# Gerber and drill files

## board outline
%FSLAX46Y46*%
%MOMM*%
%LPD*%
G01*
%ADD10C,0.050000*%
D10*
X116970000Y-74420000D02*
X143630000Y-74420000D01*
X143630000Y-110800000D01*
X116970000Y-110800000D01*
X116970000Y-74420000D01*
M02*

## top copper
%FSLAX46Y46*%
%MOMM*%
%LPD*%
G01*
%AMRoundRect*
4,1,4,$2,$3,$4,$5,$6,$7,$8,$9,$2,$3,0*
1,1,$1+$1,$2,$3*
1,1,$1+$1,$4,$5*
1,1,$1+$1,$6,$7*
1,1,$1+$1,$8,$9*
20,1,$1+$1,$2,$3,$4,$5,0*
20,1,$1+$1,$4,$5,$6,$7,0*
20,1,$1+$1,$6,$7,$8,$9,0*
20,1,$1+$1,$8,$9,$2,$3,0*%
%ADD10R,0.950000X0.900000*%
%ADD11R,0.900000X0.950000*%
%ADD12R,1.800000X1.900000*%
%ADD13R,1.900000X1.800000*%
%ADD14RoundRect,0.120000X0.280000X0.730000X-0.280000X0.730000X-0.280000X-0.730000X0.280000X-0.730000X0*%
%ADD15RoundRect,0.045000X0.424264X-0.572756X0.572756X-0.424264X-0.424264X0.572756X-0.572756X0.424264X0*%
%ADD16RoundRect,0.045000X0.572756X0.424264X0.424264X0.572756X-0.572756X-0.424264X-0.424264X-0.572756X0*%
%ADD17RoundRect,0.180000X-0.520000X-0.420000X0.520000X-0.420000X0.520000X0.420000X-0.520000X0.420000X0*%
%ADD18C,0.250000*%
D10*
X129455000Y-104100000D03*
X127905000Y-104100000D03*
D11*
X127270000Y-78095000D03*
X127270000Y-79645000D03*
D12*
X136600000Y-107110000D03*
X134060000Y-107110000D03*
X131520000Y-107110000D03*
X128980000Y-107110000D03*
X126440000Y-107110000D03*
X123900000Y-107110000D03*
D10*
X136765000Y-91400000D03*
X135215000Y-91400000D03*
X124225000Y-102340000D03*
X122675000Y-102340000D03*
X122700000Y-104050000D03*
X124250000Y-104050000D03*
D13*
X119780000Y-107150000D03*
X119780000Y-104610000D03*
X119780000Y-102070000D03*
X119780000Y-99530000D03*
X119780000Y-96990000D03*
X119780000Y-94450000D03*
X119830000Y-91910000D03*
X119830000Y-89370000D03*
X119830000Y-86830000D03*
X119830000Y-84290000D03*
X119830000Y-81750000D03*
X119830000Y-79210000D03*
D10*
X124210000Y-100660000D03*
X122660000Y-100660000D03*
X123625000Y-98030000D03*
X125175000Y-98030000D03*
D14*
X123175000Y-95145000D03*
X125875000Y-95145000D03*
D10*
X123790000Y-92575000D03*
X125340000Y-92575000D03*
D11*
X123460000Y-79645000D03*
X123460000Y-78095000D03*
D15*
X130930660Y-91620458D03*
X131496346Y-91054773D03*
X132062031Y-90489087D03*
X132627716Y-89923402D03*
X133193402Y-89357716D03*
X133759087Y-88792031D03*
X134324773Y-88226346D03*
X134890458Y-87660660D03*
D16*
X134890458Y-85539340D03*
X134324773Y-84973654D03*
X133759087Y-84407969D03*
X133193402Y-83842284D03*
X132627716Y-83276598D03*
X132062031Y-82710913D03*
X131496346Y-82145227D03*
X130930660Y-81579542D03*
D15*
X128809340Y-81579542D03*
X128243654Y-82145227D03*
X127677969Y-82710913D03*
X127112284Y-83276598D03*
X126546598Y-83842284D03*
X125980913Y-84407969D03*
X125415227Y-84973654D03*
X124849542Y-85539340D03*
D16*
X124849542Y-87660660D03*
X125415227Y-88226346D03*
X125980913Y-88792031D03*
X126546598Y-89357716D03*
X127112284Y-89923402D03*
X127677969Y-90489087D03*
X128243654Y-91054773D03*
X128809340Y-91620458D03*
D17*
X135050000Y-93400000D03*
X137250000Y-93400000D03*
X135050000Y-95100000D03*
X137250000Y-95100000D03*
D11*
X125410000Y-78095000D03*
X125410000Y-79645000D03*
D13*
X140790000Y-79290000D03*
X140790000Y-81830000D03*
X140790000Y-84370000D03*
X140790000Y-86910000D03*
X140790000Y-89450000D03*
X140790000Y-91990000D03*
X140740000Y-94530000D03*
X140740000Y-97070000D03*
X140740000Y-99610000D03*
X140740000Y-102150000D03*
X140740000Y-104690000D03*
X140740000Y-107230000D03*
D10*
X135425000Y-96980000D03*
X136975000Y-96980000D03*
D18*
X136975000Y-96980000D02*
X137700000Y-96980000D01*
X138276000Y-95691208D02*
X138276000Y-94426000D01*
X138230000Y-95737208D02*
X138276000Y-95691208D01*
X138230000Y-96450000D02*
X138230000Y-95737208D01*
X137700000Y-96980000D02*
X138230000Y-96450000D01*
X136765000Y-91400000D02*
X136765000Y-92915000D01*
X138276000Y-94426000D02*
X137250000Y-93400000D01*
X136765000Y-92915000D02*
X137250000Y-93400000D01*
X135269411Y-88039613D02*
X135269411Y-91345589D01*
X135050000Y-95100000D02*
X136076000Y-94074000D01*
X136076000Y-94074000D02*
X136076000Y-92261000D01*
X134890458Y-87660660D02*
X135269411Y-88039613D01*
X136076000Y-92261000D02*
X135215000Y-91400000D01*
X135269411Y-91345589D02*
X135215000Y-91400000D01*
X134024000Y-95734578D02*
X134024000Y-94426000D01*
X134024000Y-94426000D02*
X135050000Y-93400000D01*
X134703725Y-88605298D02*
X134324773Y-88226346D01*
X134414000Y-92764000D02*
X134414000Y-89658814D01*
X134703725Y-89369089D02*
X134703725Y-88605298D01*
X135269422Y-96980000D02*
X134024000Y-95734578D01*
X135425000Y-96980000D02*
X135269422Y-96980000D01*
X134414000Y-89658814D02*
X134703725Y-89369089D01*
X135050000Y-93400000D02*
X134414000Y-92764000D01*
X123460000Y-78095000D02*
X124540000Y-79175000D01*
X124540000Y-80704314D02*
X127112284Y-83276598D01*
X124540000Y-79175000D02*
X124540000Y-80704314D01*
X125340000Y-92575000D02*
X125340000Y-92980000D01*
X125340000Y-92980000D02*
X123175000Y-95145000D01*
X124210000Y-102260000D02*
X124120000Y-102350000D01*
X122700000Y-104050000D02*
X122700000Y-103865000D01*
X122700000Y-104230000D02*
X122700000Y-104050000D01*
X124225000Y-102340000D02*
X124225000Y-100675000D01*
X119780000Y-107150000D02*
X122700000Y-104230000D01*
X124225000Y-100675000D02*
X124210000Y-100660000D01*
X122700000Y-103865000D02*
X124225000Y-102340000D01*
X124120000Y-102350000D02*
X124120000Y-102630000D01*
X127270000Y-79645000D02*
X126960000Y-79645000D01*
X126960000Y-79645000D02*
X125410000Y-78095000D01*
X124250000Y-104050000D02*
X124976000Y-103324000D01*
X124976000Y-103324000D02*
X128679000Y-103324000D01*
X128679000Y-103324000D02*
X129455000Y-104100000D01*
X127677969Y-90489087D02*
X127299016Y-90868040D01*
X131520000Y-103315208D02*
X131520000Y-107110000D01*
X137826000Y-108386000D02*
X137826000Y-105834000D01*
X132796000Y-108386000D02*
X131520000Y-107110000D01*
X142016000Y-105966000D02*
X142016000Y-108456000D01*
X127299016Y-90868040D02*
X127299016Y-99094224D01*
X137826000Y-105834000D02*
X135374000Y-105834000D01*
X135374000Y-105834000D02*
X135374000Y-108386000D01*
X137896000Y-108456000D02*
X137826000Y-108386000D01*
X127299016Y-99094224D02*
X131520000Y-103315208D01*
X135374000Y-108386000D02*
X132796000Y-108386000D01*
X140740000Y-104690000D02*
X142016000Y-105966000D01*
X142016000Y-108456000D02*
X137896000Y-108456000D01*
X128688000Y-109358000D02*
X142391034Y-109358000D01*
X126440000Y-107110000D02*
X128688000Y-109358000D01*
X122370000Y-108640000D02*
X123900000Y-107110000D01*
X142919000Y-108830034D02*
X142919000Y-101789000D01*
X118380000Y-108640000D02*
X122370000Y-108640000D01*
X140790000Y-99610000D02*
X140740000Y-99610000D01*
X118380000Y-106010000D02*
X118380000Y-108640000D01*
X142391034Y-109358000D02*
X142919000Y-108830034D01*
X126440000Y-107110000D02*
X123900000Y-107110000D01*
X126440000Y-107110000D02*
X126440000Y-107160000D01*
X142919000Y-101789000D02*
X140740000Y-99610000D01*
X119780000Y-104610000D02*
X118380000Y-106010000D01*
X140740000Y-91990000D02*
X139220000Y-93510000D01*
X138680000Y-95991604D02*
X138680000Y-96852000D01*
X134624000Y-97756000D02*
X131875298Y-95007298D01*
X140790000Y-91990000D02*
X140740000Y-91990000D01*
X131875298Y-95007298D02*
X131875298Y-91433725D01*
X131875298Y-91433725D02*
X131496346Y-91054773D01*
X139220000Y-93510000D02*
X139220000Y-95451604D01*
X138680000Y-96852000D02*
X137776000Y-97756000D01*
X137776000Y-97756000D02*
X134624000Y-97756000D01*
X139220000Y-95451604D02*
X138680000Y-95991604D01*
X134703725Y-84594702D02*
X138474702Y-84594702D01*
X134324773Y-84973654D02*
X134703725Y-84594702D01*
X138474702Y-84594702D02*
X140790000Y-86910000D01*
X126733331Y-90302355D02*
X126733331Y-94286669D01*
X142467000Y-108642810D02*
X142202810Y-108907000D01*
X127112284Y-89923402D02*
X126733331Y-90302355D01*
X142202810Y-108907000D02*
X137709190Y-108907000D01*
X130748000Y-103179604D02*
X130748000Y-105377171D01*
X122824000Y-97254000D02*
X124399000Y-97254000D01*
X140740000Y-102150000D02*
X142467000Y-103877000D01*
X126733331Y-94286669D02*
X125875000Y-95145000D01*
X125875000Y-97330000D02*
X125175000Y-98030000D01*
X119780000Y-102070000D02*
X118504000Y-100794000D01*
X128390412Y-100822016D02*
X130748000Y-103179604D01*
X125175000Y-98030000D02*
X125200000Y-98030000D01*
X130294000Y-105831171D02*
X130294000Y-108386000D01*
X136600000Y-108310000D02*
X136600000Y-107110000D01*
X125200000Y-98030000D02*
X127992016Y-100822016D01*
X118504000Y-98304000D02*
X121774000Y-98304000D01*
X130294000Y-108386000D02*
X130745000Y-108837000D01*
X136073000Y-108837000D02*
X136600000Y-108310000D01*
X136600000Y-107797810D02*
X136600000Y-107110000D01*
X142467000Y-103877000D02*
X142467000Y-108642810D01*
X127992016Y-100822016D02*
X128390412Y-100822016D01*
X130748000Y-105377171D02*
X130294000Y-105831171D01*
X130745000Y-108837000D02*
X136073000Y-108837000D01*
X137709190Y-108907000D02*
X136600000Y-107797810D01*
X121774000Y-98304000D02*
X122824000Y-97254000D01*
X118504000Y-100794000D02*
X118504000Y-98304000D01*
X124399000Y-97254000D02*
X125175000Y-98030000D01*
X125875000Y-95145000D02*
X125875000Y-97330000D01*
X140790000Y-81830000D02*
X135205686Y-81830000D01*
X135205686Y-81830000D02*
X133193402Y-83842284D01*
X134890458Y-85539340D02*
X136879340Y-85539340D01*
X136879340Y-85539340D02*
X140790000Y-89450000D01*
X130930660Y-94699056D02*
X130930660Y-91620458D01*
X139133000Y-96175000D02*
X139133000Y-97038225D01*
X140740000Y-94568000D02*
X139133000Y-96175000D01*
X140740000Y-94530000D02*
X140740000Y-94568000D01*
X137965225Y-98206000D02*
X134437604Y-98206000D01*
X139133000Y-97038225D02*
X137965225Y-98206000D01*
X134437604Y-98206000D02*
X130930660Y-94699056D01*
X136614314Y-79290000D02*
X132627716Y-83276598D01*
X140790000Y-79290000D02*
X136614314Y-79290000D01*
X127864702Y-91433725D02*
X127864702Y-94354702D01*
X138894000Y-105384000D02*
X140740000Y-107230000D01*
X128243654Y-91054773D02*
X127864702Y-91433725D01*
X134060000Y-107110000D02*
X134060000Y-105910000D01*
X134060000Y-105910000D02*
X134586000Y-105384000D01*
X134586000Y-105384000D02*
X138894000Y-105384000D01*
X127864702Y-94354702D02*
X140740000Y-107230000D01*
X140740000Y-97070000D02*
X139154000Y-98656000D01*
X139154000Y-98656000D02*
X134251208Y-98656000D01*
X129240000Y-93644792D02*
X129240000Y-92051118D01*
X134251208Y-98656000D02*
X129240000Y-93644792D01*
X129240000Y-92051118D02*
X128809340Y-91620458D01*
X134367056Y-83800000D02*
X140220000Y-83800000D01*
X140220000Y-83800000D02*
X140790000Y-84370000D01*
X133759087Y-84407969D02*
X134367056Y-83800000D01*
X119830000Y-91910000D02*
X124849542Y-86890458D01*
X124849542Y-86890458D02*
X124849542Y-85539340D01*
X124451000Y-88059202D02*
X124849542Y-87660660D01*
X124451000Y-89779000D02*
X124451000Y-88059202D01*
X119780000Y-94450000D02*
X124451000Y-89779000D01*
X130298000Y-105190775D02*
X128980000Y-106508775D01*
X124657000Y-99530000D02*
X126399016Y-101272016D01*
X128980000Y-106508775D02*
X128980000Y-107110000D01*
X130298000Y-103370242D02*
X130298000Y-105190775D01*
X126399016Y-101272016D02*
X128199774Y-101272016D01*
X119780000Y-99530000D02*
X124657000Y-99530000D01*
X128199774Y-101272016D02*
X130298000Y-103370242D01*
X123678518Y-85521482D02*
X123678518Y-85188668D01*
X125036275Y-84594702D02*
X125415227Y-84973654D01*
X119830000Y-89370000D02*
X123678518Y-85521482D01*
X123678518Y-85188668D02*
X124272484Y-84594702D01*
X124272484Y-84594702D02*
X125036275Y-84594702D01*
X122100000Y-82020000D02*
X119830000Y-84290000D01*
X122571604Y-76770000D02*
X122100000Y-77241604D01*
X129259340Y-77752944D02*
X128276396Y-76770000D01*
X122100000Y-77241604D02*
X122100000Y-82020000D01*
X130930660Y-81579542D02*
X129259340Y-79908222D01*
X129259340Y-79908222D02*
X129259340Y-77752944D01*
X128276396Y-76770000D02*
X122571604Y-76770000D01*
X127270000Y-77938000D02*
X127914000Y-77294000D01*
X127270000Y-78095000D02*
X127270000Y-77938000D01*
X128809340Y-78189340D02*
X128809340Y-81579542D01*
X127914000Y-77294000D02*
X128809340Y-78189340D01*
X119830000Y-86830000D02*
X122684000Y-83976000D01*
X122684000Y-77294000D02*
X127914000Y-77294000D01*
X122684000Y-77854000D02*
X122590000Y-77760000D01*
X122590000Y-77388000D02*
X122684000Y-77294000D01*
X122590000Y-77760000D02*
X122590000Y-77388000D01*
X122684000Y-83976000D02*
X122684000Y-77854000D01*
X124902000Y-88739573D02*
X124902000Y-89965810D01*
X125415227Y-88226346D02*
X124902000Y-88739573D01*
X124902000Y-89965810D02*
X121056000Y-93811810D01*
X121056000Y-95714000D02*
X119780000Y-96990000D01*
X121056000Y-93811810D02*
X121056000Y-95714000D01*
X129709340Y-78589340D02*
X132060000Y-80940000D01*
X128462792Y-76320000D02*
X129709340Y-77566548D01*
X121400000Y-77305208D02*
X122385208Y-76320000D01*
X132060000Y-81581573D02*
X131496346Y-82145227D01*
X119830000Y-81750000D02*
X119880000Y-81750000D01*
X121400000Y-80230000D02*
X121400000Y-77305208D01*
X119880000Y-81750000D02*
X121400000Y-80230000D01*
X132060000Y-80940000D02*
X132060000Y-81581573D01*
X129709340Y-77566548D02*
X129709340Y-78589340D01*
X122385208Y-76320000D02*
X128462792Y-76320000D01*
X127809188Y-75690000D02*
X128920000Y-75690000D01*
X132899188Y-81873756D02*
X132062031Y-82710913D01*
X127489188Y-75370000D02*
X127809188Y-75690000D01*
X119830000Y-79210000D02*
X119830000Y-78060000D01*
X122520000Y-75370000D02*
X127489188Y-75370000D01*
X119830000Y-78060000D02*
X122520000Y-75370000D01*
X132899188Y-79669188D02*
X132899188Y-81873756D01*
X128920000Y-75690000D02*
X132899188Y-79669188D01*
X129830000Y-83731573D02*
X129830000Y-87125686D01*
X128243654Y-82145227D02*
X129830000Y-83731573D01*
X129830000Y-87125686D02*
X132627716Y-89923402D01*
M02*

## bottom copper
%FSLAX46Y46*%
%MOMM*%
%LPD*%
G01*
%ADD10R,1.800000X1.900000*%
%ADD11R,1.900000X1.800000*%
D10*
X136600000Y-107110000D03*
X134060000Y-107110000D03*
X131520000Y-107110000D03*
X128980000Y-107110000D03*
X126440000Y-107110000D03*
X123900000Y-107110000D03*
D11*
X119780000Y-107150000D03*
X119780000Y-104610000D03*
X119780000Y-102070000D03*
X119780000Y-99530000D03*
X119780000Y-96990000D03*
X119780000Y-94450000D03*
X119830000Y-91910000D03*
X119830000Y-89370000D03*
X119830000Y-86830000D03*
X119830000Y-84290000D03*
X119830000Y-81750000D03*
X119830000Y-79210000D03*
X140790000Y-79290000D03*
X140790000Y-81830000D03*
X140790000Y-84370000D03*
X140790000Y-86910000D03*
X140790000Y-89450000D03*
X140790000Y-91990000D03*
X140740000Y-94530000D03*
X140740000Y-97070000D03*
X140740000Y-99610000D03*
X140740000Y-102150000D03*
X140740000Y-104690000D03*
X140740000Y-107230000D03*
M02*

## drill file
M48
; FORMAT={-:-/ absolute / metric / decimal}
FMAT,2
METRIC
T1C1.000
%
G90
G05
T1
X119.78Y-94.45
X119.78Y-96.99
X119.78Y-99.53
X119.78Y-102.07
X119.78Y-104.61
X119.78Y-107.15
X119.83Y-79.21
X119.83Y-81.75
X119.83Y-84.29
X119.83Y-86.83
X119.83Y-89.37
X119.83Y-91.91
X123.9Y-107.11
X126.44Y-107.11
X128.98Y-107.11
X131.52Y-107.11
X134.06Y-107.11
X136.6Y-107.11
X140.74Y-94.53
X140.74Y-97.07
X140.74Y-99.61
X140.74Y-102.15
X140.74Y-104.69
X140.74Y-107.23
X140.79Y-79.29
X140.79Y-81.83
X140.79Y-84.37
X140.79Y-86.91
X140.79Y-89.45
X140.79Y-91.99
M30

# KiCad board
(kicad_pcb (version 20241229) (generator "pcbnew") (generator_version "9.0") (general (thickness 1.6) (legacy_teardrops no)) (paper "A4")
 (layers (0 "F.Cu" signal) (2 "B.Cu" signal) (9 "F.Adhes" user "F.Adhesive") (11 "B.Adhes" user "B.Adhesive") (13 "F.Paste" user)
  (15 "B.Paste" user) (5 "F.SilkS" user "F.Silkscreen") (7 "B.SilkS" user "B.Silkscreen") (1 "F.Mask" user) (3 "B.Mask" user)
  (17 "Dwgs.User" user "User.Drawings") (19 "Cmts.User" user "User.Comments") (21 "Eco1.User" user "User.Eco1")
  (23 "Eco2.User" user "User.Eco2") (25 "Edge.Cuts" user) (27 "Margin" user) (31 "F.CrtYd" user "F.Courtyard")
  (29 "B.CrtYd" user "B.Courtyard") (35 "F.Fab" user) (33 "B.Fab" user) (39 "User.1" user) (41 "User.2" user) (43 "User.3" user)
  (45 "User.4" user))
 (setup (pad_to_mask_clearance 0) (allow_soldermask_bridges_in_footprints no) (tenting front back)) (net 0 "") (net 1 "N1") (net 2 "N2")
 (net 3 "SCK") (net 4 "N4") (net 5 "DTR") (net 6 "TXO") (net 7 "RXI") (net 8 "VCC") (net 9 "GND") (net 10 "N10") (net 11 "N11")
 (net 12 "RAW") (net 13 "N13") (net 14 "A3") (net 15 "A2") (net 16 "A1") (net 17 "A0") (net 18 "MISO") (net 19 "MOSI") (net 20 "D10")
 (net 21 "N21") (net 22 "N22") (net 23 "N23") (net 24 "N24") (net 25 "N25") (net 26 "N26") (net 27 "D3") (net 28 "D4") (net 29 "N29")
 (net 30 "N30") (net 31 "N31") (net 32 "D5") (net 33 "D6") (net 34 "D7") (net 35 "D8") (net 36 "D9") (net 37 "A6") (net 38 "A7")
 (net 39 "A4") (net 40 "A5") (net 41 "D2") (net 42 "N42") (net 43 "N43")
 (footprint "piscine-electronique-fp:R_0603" (layer "F.Cu") (at 128.68 104.1 180)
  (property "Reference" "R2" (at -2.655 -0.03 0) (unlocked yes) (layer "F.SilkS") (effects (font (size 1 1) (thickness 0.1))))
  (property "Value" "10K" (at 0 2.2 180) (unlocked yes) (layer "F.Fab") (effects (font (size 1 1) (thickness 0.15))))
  (pad "1" smd rect (at -0.775 0 180) (size 0.95 0.9) (layers "F.Cu" "F.Mask" "F.Paste") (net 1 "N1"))
  (pad "2" smd rect (at 0.775 0 180) (size 0.95 0.9) (layers "F.Cu" "F.Mask" "F.Paste") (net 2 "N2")))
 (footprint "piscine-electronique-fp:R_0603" (layer "F.Cu") (at 127.27 78.87 -90)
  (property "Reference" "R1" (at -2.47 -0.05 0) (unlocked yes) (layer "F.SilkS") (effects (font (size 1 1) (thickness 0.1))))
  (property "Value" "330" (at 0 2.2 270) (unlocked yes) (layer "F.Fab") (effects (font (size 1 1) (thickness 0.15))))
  (pad "1" smd rect (at -0.775 0 270) (size 0.95 0.9) (layers "F.Cu" "F.Mask" "F.Paste") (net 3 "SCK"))
  (pad "2" smd rect (at 0.775 0 270) (size 0.95 0.9) (layers "F.Cu" "F.Mask" "F.Paste") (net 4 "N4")))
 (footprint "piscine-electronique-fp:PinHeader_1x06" (layer "F.Cu") (at 130.25 107.11 -90)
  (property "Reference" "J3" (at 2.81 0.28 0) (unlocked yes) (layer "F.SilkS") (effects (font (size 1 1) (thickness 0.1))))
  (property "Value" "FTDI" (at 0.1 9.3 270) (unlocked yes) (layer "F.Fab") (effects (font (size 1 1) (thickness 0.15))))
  (pad "1" thru_hole rect (at 0 -6.35 270) (size 1.9 1.8) (drill 1) (layers "*.Cu" "*.Mask") (remove_unused_layers no) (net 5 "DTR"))
  (pad "2" thru_hole rect (at 0 -3.81 270) (size 1.9 1.8) (drill 1) (layers "*.Cu" "*.Mask") (remove_unused_layers no) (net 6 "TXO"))
  (pad "3" thru_hole rect (at 0 -1.27 270) (size 1.9 1.8) (drill 1) (layers "*.Cu" "*.Mask") (remove_unused_layers no) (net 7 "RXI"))
  (pad "4" thru_hole rect (at 0 1.27 270) (size 1.9 1.8) (drill 1) (layers "*.Cu" "*.Mask") (remove_unused_layers no) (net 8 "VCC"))
  (pad "5" thru_hole rect (at 0 3.81 270) (size 1.9 1.8) (drill 1) (layers "*.Cu" "*.Mask") (remove_unused_layers no) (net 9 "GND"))
  (pad "6" thru_hole rect (at 0 6.35 270) (size 1.9 1.8) (drill 1) (layers "*.Cu" "*.Mask") (remove_unused_layers no) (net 9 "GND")))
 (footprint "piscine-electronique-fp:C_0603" (layer "F.Cu") (at 135.99 91.4 180)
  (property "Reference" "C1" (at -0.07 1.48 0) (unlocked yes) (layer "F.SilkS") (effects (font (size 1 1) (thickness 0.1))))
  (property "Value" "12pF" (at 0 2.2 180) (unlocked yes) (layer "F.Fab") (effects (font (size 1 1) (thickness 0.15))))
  (pad "1" smd rect (at -0.775 0 180) (size 0.95 0.9) (layers "F.Cu" "F.Mask" "F.Paste") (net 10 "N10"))
  (pad "2" smd rect (at 0.775 0 180) (size 0.95 0.9) (layers "F.Cu" "F.Mask" "F.Paste") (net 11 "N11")))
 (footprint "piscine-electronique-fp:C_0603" (layer "F.Cu") (at 123.45 102.34 180)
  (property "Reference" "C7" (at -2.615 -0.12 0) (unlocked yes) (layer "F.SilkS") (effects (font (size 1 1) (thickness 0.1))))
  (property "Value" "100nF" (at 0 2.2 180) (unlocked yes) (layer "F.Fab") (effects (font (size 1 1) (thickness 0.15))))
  (pad "1" smd rect (at -0.775 0 180) (size 0.95 0.9) (layers "F.Cu" "F.Mask" "F.Paste") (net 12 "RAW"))
  (pad "2" smd rect (at 0.775 0 180) (size 0.95 0.9) (layers "F.Cu" "F.Mask" "F.Paste") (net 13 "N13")))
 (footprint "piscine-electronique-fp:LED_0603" (layer "F.Cu") (at 123.475 104.05)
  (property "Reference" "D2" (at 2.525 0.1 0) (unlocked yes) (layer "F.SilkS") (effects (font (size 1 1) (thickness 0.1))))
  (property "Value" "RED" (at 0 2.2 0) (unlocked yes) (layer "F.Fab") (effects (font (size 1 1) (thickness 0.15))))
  (pad "1" smd rect (at -0.775 0) (size 0.95 0.9) (layers "F.Cu" "F.Mask" "F.Paste") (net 12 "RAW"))
  (pad "2" smd rect (at 0.775 0) (size 0.95 0.9) (layers "F.Cu" "F.Mask" "F.Paste") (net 1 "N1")))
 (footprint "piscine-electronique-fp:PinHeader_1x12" (layer "F.Cu") (at 119.83 93.18 180)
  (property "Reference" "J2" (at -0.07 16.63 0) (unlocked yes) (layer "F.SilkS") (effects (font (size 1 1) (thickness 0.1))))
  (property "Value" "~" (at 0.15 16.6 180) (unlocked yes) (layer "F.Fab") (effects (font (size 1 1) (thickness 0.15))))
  (pad "1" thru_hole rect (at 0.05 -13.97 180) (size 1.9 1.8) (drill 1) (layers "*.Cu" "*.Mask") (remove_unused_layers no) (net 12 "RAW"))
  (pad "2" thru_hole rect (at 0.05 -11.43 180) (size 1.9 1.8) (drill 1) (layers "*.Cu" "*.Mask") (remove_unused_layers no) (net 9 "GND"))
  (pad "3" thru_hole rect (at 0.05 -8.89 180) (size 1.9 1.8) (drill 1) (layers "*.Cu" "*.Mask") (remove_unused_layers no) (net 5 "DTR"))
  (pad "4" thru_hole rect (at 0.05 -6.35 180) (size 1.9 1.8) (drill 1) (layers "*.Cu" "*.Mask") (remove_unused_layers no) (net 8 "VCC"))
  (pad "5" thru_hole rect (at 0.05 -3.81 180) (size 1.9 1.8) (drill 1) (layers "*.Cu" "*.Mask") (remove_unused_layers no) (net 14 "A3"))
  (pad "6" thru_hole rect (at 0.05 -1.27 180) (size 1.9 1.8) (drill 1) (layers "*.Cu" "*.Mask") (remove_unused_layers no) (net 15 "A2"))
  (pad "7" thru_hole rect (at 0 1.27 180) (size 1.9 1.8) (drill 1) (layers "*.Cu" "*.Mask") (remove_unused_layers no) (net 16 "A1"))
  (pad "8" thru_hole rect (at 0 3.81 180) (size 1.9 1.8) (drill 1) (layers "*.Cu" "*.Mask") (remove_unused_layers no) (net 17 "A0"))
  (pad "9" thru_hole rect (at 0 6.35 180) (size 1.9 1.8) (drill 1) (layers "*.Cu" "*.Mask") (remove_unused_layers no) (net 3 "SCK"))
  (pad "10" thru_hole rect (at 0 8.89 180) (size 1.9 1.8) (drill 1) (layers "*.Cu" "*.Mask") (remove_unused_layers no) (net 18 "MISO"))
  (pad "11" thru_hole rect (at 0 11.43 180) (size 1.9 1.8) (drill 1) (layers "*.Cu" "*.Mask") (remove_unused_layers no) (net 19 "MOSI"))
  (pad "12" thru_hole rect (at 0 13.97 180) (size 1.9 1.8) (drill 1) (layers "*.Cu" "*.Mask") (remove_unused_layers no) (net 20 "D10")))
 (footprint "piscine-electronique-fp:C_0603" (layer "F.Cu") (at 123.435 100.66 180)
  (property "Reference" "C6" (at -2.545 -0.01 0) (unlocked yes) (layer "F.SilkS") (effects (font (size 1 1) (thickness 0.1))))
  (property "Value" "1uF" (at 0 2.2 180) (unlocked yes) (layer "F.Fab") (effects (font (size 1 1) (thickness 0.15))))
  (pad "1" smd rect (at -0.775 0 180) (size 0.95 0.9) (layers "F.Cu" "F.Mask" "F.Paste") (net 12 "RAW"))
  (pad "2" smd rect (at 0.775 0 180) (size 0.95 0.9) (layers "F.Cu" "F.Mask" "F.Paste") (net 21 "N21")))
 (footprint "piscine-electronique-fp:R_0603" (layer "F.Cu") (at 124.4 98.03)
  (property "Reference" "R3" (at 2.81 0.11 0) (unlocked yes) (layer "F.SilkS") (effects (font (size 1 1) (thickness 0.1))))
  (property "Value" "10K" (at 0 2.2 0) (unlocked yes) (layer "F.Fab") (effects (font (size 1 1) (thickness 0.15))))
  (pad "1" smd rect (at -0.775 0) (size 0.95 0.9) (layers "F.Cu" "F.Mask" "F.Paste") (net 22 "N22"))
  (pad "2" smd rect (at 0.775 0) (size 0.95 0.9) (layers "F.Cu" "F.Mask" "F.Paste") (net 5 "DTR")))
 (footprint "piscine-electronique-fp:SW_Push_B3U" (layer "F.Cu") (at 124.525 95.145)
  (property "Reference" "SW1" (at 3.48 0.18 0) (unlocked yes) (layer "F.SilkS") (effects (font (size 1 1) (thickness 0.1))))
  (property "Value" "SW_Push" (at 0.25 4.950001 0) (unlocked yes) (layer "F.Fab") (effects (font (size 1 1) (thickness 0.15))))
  (pad "1" smd roundrect (at -1.35 0 180) (size 0.8 1.7) (layers "F.Cu" "F.Mask" "F.Paste") (roundrect_rratio 0.15) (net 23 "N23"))
  (pad "2" smd roundrect (at 1.35 0 180) (size 0.8 1.7) (layers "F.Cu" "F.Mask" "F.Paste") (roundrect_rratio 0.15) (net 5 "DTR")))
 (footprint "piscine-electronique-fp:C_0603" (layer "F.Cu") (at 124.565 92.575)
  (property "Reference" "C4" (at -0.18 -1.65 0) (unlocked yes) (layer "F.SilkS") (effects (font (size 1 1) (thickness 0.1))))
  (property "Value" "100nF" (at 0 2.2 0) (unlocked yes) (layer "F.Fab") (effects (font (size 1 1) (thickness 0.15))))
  (pad "1" smd rect (at -0.775 0) (size 0.95 0.9) (layers "F.Cu" "F.Mask" "F.Paste") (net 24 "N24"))
  (pad "2" smd rect (at 0.775 0) (size 0.95 0.9) (layers "F.Cu" "F.Mask" "F.Paste") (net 23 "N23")))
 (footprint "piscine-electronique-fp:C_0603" (layer "F.Cu") (at 123.46 78.87 90)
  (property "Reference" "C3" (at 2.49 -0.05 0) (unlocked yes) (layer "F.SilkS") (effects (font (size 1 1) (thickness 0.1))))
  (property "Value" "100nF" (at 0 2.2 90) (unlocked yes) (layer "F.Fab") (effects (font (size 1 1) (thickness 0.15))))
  (pad "1" smd rect (at -0.775 0 90) (size 0.95 0.9) (layers "F.Cu" "F.Mask" "F.Paste") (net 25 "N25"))
  (pad "2" smd rect (at 0.775 0 90) (size 0.95 0.9) (layers "F.Cu" "F.Mask" "F.Paste") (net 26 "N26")))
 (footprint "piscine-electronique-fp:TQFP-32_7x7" (layer "F.Cu") (at 129.87 86.6 135)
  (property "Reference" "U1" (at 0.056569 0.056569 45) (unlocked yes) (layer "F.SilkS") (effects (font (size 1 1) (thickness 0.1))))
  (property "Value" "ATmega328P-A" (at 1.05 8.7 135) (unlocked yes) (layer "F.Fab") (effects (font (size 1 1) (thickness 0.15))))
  (pad "1" smd roundrect (at -4.3 -2.8 45) (size 0.3 1.5) (layers "F.Cu" "F.Mask" "F.Paste") (roundrect_rratio 0.15) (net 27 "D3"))
  (pad "2" smd roundrect (at -4.3 -2 45) (size 0.3 1.5) (layers "F.Cu" "F.Mask" "F.Paste") (roundrect_rratio 0.15) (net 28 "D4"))
  (pad "3" smd roundrect (at -4.3 -1.2 45) (size 0.3 1.5) (layers "F.Cu" "F.Mask" "F.Paste") (roundrect_rratio 0.15) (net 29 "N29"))
  (pad "4" smd roundrect (at -4.3 -0.4 45) (size 0.3 1.5) (layers "F.Cu" "F.Mask" "F.Paste") (roundrect_rratio 0.15) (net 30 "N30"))
  (pad "5" smd roundrect (at -4.3 0.4 45) (size 0.3 1.5) (layers "F.Cu" "F.Mask" "F.Paste") (roundrect_rratio 0.15))
  (pad "6" smd roundrect (at -4.3 1.2 45) (size 0.3 1.5) (layers "F.Cu" "F.Mask" "F.Paste") (roundrect_rratio 0.15))
  (pad "7" smd roundrect (at -4.3 2 45) (size 0.3 1.5) (layers "F.Cu" "F.Mask" "F.Paste") (roundrect_rratio 0.15) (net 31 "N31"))
  (pad "8" smd roundrect (at -4.3 2.8 45) (size 0.3 1.5) (layers "F.Cu" "F.Mask" "F.Paste") (roundrect_rratio 0.15) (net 11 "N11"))
  (pad "9" smd roundrect (at -2.8 4.3 135) (size 0.3 1.5) (layers "F.Cu" "F.Mask" "F.Paste") (roundrect_rratio 0.15) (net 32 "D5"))
  (pad "10" smd roundrect (at -2 4.3 135) (size 0.3 1.5) (layers "F.Cu" "F.Mask" "F.Paste") (roundrect_rratio 0.15) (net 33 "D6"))
  (pad "11" smd roundrect (at -1.2 4.3 135) (size 0.3 1.5) (layers "F.Cu" "F.Mask" "F.Paste") (roundrect_rratio 0.15) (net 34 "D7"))
  (pad "12" smd roundrect (at -0.4 4.3 135) (size 0.3 1.5) (layers "F.Cu" "F.Mask" "F.Paste") (roundrect_rratio 0.15) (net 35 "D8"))
  (pad "13" smd roundrect (at 0.4 4.3 135) (size 0.3 1.5) (layers "F.Cu" "F.Mask" "F.Paste") (roundrect_rratio 0.15) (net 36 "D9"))
  (pad "14" smd roundrect (at 1.2 4.3 135) (size 0.3 1.5) (layers "F.Cu" "F.Mask" "F.Paste") (roundrect_rratio 0.15) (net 20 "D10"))
  (pad "15" smd roundrect (at 2 4.3 135) (size 0.3 1.5) (layers "F.Cu" "F.Mask" "F.Paste") (roundrect_rratio 0.15) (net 19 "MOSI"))
  (pad "16" smd roundrect (at 2.8 4.3 135) (size 0.3 1.5) (layers "F.Cu" "F.Mask" "F.Paste") (roundrect_rratio 0.15) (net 18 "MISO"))
  (pad "17" smd roundrect (at 4.3 2.8 45) (size 0.3 1.5) (layers "F.Cu" "F.Mask" "F.Paste") (roundrect_rratio 0.15) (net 3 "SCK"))
  (pad "18" smd roundrect (at 4.3 2 45) (size 0.3 1.5) (layers "F.Cu" "F.Mask" "F.Paste") (roundrect_rratio 0.15) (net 30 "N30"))
  (pad "19" smd roundrect (at 4.3 1.2 45) (size 0.3 1.5) (layers "F.Cu" "F.Mask" "F.Paste") (roundrect_rratio 0.15) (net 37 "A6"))
  (pad "20" smd roundrect (at 4.3 0.4 45) (size 0.3 1.5) (layers "F.Cu" "F.Mask" "F.Paste") (roundrect_rratio 0.15) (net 26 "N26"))
  (pad "21" smd roundrect (at 4.3 -0.4 45) (size 0.3 1.5) (layers "F.Cu" "F.Mask" "F.Paste") (roundrect_rratio 0.15))
  (pad "22" smd roundrect (at 4.3 -1.2 45) (size 0.3 1.5) (layers "F.Cu" "F.Mask" "F.Paste") (roundrect_rratio 0.15) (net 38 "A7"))
  (pad "23" smd roundrect (at 4.3 -2 45) (size 0.3 1.5) (layers "F.Cu" "F.Mask" "F.Paste") (roundrect_rratio 0.15) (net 17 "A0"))
  (pad "24" smd roundrect (at 4.3 -2.8 45) (size 0.3 1.5) (layers "F.Cu" "F.Mask" "F.Paste") (roundrect_rratio 0.15) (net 16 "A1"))
  (pad "25" smd roundrect (at 2.8 -4.3 135) (size 0.3 1.5) (layers "F.Cu" "F.Mask" "F.Paste") (roundrect_rratio 0.15) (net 15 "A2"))
  (pad "26" smd roundrect (at 2 -4.3 135) (size 0.3 1.5) (layers "F.Cu" "F.Mask" "F.Paste") (roundrect_rratio 0.15) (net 14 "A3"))
  (pad "27" smd roundrect (at 1.2 -4.3 135) (size 0.3 1.5) (layers "F.Cu" "F.Mask" "F.Paste") (roundrect_rratio 0.15) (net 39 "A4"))
  (pad "28" smd roundrect (at 0.4 -4.3 135) (size 0.3 1.5) (layers "F.Cu" "F.Mask" "F.Paste") (roundrect_rratio 0.15) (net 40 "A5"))
  (pad "29" smd roundrect (at -0.4 -4.3 135) (size 0.3 1.5) (layers "F.Cu" "F.Mask" "F.Paste") (roundrect_rratio 0.15) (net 5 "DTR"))
  (pad "30" smd roundrect (at -1.2 -4.3 135) (size 0.3 1.5) (layers "F.Cu" "F.Mask" "F.Paste") (roundrect_rratio 0.15) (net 7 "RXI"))
  (pad "31" smd roundrect (at -2 -4.3 135) (size 0.3 1.5) (layers "F.Cu" "F.Mask" "F.Paste") (roundrect_rratio 0.15) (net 6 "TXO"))
  (pad "32" smd roundrect (at -2.8 -4.3 135) (size 0.3 1.5) (layers "F.Cu" "F.Mask" "F.Paste") (roundrect_rratio 0.15) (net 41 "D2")))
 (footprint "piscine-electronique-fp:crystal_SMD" (layer "F.Cu") (at 136.15 94.25)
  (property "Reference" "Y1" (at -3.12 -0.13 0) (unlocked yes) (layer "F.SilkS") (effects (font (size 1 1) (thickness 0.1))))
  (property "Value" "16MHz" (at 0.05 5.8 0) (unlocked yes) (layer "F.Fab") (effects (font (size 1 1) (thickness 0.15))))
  (pad "1" smd roundrect (at -1.1 -0.85) (size 1.4 1.2) (layers "F.Cu" "F.Mask" "F.Paste") (roundrect_rratio 0.15) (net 31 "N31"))
  (pad "2" smd roundrect (at 1.1 -0.85) (size 1.4 1.2) (layers "F.Cu" "F.Mask" "F.Paste") (roundrect_rratio 0.15) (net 10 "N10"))
  (pad "3" smd roundrect (at -1.1 0.85) (size 1.4 1.2) (layers "F.Cu" "F.Mask" "F.Paste") (roundrect_rratio 0.15) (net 11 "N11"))
  (pad "4" smd roundrect (at 1.1 0.85) (size 1.4 1.2) (layers "F.Cu" "F.Mask" "F.Paste") (roundrect_rratio 0.15) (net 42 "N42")))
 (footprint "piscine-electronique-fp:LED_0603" (layer "F.Cu") (at 125.41 78.87 -90)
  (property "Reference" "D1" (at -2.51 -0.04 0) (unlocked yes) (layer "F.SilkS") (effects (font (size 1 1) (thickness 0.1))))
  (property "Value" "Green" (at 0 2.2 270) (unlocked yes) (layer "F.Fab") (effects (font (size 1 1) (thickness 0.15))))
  (pad "1" smd rect (at -0.775 0 270) (size 0.95 0.9) (layers "F.Cu" "F.Mask" "F.Paste") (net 4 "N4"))
  (pad "2" smd rect (at 0.775 0 270) (size 0.95 0.9) (layers "F.Cu" "F.Mask" "F.Paste") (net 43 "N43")))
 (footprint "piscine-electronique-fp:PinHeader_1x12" (layer "F.Cu") (at 140.74 93.26)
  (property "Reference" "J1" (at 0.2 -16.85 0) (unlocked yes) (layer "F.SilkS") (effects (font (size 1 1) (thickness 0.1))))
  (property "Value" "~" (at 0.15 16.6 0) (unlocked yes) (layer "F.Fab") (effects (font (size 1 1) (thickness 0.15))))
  (pad "1" thru_hole rect (at 0.05 -13.97) (size 1.9 1.8) (drill 1) (layers "*.Cu" "*.Mask") (remove_unused_layers no) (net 36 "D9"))
  (pad "2" thru_hole rect (at 0.05 -11.43) (size 1.9 1.8) (drill 1) (layers "*.Cu" "*.Mask") (remove_unused_layers no) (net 35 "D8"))
  (pad "3" thru_hole rect (at 0.05 -8.89) (size 1.9 1.8) (drill 1) (layers "*.Cu" "*.Mask") (remove_unused_layers no) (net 34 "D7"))
  (pad "4" thru_hole rect (at 0.05 -6.35) (size 1.9 1.8) (drill 1) (layers "*.Cu" "*.Mask") (remove_unused_layers no) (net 33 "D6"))
  (pad "5" thru_hole rect (at 0.05 -3.81) (size 1.9 1.8) (drill 1) (layers "*.Cu" "*.Mask") (remove_unused_layers no) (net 32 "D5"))
  (pad "6" thru_hole rect (at 0.05 -1.27) (size 1.9 1.8) (drill 1) (layers "*.Cu" "*.Mask") (remove_unused_layers no) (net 28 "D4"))
  (pad "7" thru_hole rect (at 0 1.27) (size 1.9 1.8) (drill 1) (layers "*.Cu" "*.Mask") (remove_unused_layers no) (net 27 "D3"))
  (pad "8" thru_hole rect (at 0 3.81) (size 1.9 1.8) (drill 1) (layers "*.Cu" "*.Mask") (remove_unused_layers no) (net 41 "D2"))
  (pad "9" thru_hole rect (at 0 6.35) (size 1.9 1.8) (drill 1) (layers "*.Cu" "*.Mask") (remove_unused_layers no) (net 9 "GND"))
  (pad "10" thru_hole rect (at 0 8.89) (size 1.9 1.8) (drill 1) (layers "*.Cu" "*.Mask") (remove_unused_layers no) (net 5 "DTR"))
  (pad "11" thru_hole rect (at 0 11.43) (size 1.9 1.8) (drill 1) (layers "*.Cu" "*.Mask") (remove_unused_layers no) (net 7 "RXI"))
  (pad "12" thru_hole rect (at 0 13.97) (size 1.9 1.8) (drill 1) (layers "*.Cu" "*.Mask") (remove_unused_layers no) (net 6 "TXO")))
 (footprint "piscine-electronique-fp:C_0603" (layer "F.Cu") (at 136.2 96.98)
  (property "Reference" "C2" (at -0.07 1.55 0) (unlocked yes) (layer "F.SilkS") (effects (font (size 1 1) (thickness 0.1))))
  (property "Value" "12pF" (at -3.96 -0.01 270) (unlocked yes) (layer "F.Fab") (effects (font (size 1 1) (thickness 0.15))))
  (pad "1" smd rect (at -0.775 0) (size 0.95 0.9) (layers "F.Cu" "F.Mask" "F.Paste") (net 31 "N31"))
  (pad "2" smd rect (at 0.775 0) (size 0.95 0.9) (layers "F.Cu" "F.Mask" "F.Paste") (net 10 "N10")))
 (gr_rect (start 116.97 74.42) (end 143.63 110.8) (stroke (width 0.05) (type default)) (fill no) (layer "Edge.Cuts"))
 (segment (start 136.975 96.98) (end 137.7 96.98) (width 0.25) (layer "F.Cu") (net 10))
 (segment (start 138.276 95.691208) (end 138.276 94.426) (width 0.25) (layer "F.Cu") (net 10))
 (segment (start 138.23 95.737208) (end 138.276 95.691208) (width 0.25) (layer "F.Cu") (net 10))
 (segment (start 138.23 96.45) (end 138.23 95.737208) (width 0.25) (layer "F.Cu") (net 10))
 (segment (start 137.7 96.98) (end 138.23 96.45) (width 0.25) (layer "F.Cu") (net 10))
 (segment (start 136.765 91.4) (end 136.765 92.915) (width 0.25) (layer "F.Cu") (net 10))
 (segment (start 138.276 94.426) (end 137.25 93.4) (width 0.25) (layer "F.Cu") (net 10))
 (segment (start 136.765 92.915) (end 137.25 93.4) (width 0.25) (layer "F.Cu") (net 10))
 (segment (start 135.269411 88.039613) (end 135.269411 91.345589) (width 0.25) (layer "F.Cu") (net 11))
 (segment (start 135.05 95.1) (end 136.076 94.074) (width 0.25) (layer "F.Cu") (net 11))
 (segment (start 136.076 94.074) (end 136.076 92.261) (width 0.25) (layer "F.Cu") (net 11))
 (segment (start 134.890458 87.66066) (end 135.269411 88.039613) (width 0.25) (layer "F.Cu") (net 11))
 (segment (start 136.076 92.261) (end 135.215 91.4) (width 0.25) (layer "F.Cu") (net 11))
 (segment (start 135.269411 91.345589) (end 135.215 91.4) (width 0.25) (layer "F.Cu") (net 11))
 (segment (start 134.024 95.734578) (end 134.024 94.426) (width 0.25) (layer "F.Cu") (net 31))
 (segment (start 134.024 94.426) (end 135.05 93.4) (width 0.25) (layer "F.Cu") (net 31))
 (segment (start 134.703725 88.605298) (end 134.324773 88.226346) (width 0.25) (layer "F.Cu") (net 31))
 (segment (start 134.414 92.764) (end 134.414 89.658814) (width 0.25) (layer "F.Cu") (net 31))
 (segment (start 134.703725 89.369089) (end 134.703725 88.605298) (width 0.25) (layer "F.Cu") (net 31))
 (segment (start 135.269422 96.98) (end 134.024 95.734578) (width 0.25) (layer "F.Cu") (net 31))
 (segment (start 135.425 96.98) (end 135.269422 96.98) (width 0.25) (layer "F.Cu") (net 31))
 (segment (start 134.414 89.658814) (end 134.703725 89.369089) (width 0.25) (layer "F.Cu") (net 31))
 (segment (start 135.05 93.4) (end 134.414 92.764) (width 0.25) (layer "F.Cu") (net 31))
 (segment (start 123.46 78.095) (end 124.54 79.175) (width 0.25) (layer "F.Cu") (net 26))
 (segment (start 124.54 80.704314) (end 127.112284 83.276598) (width 0.25) (layer "F.Cu") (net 26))
 (segment (start 124.54 79.175) (end 124.54 80.704314) (width 0.25) (layer "F.Cu") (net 26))
 (segment (start 125.34 92.575) (end 125.34 92.98) (width 0.25) (layer "F.Cu") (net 23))
 (segment (start 125.34 92.98) (end 123.175 95.145) (width 0.25) (layer "F.Cu") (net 23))
 (segment (start 124.21 102.26) (end 124.12 102.35) (width 0.25) (layer "F.Cu") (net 12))
 (segment (start 122.7 104.05) (end 122.7 103.865) (width 0.25) (layer "F.Cu") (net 12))
 (segment (start 122.7 104.23) (end 122.7 104.05) (width 0.25) (layer "F.Cu") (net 12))
 (segment (start 124.225 102.34) (end 124.225 100.675) (width 0.25) (layer "F.Cu") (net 12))
 (segment (start 119.78 107.15) (end 122.7 104.23) (width 0.25) (layer "F.Cu") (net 12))
 (segment (start 124.225 100.675) (end 124.21 100.66) (width 0.25) (layer "F.Cu") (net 12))
 (segment (start 122.7 103.865) (end 124.225 102.34) (width 0.25) (layer "F.Cu") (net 12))
 (segment (start 124.12 102.35) (end 124.12 102.63) (width 0.25) (layer "F.Cu") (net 12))
 (segment (start 127.27 79.645) (end 126.96 79.645) (width 0.25) (layer "F.Cu") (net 4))
 (segment (start 126.96 79.645) (end 125.41 78.095) (width 0.25) (layer "F.Cu") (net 4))
 (segment (start 124.25 104.05) (end 124.976 103.324) (width 0.25) (layer "F.Cu") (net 1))
 (segment (start 124.976 103.324) (end 128.679 103.324) (width 0.25) (layer "F.Cu") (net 1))
 (segment (start 128.679 103.324) (end 129.455 104.1) (width 0.25) (layer "F.Cu") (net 1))
 (segment (start 127.677969 90.489087) (end 127.299016 90.86804) (width 0.25) (layer "F.Cu") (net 7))
 (segment (start 131.52 103.315208) (end 131.52 107.11) (width 0.25) (layer "F.Cu") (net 7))
 (segment (start 137.826 108.386) (end 137.826 105.834) (width 0.25) (layer "F.Cu") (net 7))
 (segment (start 132.796 108.386) (end 131.52 107.11) (width 0.25) (layer "F.Cu") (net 7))
 (segment (start 142.016 105.966) (end 142.016 108.456) (width 0.25) (layer "F.Cu") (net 7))
 (segment (start 127.299016 90.86804) (end 127.299016 99.094224) (width 0.25) (layer "F.Cu") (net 7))
 (segment (start 137.826 105.834) (end 135.374 105.834) (width 0.25) (layer "F.Cu") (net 7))
 (segment (start 135.374 105.834) (end 135.374 108.386) (width 0.25) (layer "F.Cu") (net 7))
 (segment (start 137.896 108.456) (end 137.826 108.386) (width 0.25) (layer "F.Cu") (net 7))
 (segment (start 127.299016 99.094224) (end 131.52 103.315208) (width 0.25) (layer "F.Cu") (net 7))
 (segment (start 135.374 108.386) (end 132.796 108.386) (width 0.25) (layer "F.Cu") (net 7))
 (segment (start 140.74 104.69) (end 142.016 105.966) (width 0.25) (layer "F.Cu") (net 7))
 (segment (start 142.016 108.456) (end 137.896 108.456) (width 0.25) (layer "F.Cu") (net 7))
 (segment (start 128.688 109.358) (end 142.391034 109.358) (width 0.25) (layer "F.Cu") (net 9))
 (segment (start 126.44 107.11) (end 128.688 109.358) (width 0.25) (layer "F.Cu") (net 9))
 (segment (start 122.37 108.64) (end 123.9 107.11) (width 0.25) (layer "F.Cu") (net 9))
 (segment (start 142.919 108.830034) (end 142.919 101.789) (width 0.25) (layer "F.Cu") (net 9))
 (segment (start 118.38 108.64) (end 122.37 108.64) (width 0.25) (layer "F.Cu") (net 9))
 (segment (start 140.79 99.61) (end 140.74 99.61) (width 0.25) (layer "F.Cu") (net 9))
 (segment (start 118.38 106.01) (end 118.38 108.64) (width 0.25) (layer "F.Cu") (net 9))
 (segment (start 142.391034 109.358) (end 142.919 108.830034) (width 0.25) (layer "F.Cu") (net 9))
 (segment (start 126.44 107.11) (end 123.9 107.11) (width 0.25) (layer "F.Cu") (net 9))
 (segment (start 126.44 107.11) (end 126.44 107.16) (width 0.25) (layer "F.Cu") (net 9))
 (segment (start 142.919 101.789) (end 140.74 99.61) (width 0.25) (layer "F.Cu") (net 9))
 (segment (start 119.78 104.61) (end 118.38 106.01) (width 0.25) (layer "F.Cu") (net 9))
 (segment (start 140.74 91.99) (end 139.22 93.51) (width 0.25) (layer "F.Cu") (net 28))
 (segment (start 138.68 95.991604) (end 138.68 96.852) (width 0.25) (layer "F.Cu") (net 28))
 (segment (start 134.624 97.756) (end 131.875298 95.007298) (width 0.25) (layer "F.Cu") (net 28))
 (segment (start 140.79 91.99) (end 140.74 91.99) (width 0.25) (layer "F.Cu") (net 28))
 (segment (start 131.875298 95.007298) (end 131.875298 91.433725) (width 0.25) (layer "F.Cu") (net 28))
 (segment (start 131.875298 91.433725) (end 131.496346 91.054773) (width 0.25) (layer "F.Cu") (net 28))
 (segment (start 139.22 93.51) (end 139.22 95.451604) (width 0.25) (layer "F.Cu") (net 28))
 (segment (start 138.68 96.852) (end 137.776 97.756) (width 0.25) (layer "F.Cu") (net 28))
 (segment (start 137.776 97.756) (end 134.624 97.756) (width 0.25) (layer "F.Cu") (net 28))
 (segment (start 139.22 95.451604) (end 138.68 95.991604) (width 0.25) (layer "F.Cu") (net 28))
 (segment (start 134.703725 84.594702) (end 138.474702 84.594702) (width 0.25) (layer "F.Cu") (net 33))
 (segment (start 134.324773 84.973654) (end 134.703725 84.594702) (width 0.25) (layer "F.Cu") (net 33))
 (segment (start 138.474702 84.594702) (end 140.79 86.91) (width 0.25) (layer "F.Cu") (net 33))
 (segment (start 126.733331 90.302355) (end 126.733331 94.286669) (width 0.25) (layer "F.Cu") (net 5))
 (segment (start 142.467 108.64281) (end 142.20281 108.907) (width 0.25) (layer "F.Cu") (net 5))
 (segment (start 127.112284 89.923402) (end 126.733331 90.302355) (width 0.25) (layer "F.Cu") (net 5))
 (segment (start 142.20281 108.907) (end 137.70919 108.907) (width 0.25) (layer "F.Cu") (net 5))
 (segment (start 130.748 103.179604) (end 130.748 105.377171) (width 0.25) (layer "F.Cu") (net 5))
 (segment (start 122.824 97.254) (end 124.399 97.254) (width 0.25) (layer "F.Cu") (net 5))
 (segment (start 140.74 102.15) (end 142.467 103.877) (width 0.25) (layer "F.Cu") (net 5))
 (segment (start 126.733331 94.286669) (end 125.875 95.145) (width 0.25) (layer "F.Cu") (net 5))
 (segment (start 125.875 97.33) (end 125.175 98.03) (width 0.25) (layer "F.Cu") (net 5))
 (segment (start 119.78 102.07) (end 118.504 100.794) (width 0.25) (layer "F.Cu") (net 5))
 (segment (start 128.390412 100.822016) (end 130.748 103.179604) (width 0.25) (layer "F.Cu") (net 5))
 (segment (start 125.175 98.03) (end 125.2 98.03) (width 0.25) (layer "F.Cu") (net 5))
 (segment (start 130.294 105.831171) (end 130.294 108.386) (width 0.25) (layer "F.Cu") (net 5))
 (segment (start 136.6 108.31) (end 136.6 107.11) (width 0.25) (layer "F.Cu") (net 5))
 (segment (start 125.2 98.03) (end 127.992016 100.822016) (width 0.25) (layer "F.Cu") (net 5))
 (segment (start 118.504 98.304) (end 121.774 98.304) (width 0.25) (layer "F.Cu") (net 5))
 (segment (start 130.294 108.386) (end 130.745 108.837) (width 0.25) (layer "F.Cu") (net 5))
 (segment (start 136.073 108.837) (end 136.6 108.31) (width 0.25) (layer "F.Cu") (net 5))
 (segment (start 136.6 107.79781) (end 136.6 107.11) (width 0.25) (layer "F.Cu") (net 5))
 (segment (start 142.467 103.877) (end 142.467 108.64281) (width 0.25) (layer "F.Cu") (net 5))
 (segment (start 127.992016 100.822016) (end 128.390412 100.822016) (width 0.25) (layer "F.Cu") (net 5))
 (segment (start 130.748 105.377171) (end 130.294 105.831171) (width 0.25) (layer "F.Cu") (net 5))
 (segment (start 130.745 108.837) (end 136.073 108.837) (width 0.25) (layer "F.Cu") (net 5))
 (segment (start 137.70919 108.907) (end 136.6 107.79781) (width 0.25) (layer "F.Cu") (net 5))
 (segment (start 121.774 98.304) (end 122.824 97.254) (width 0.25) (layer "F.Cu") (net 5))
 (segment (start 118.504 100.794) (end 118.504 98.304) (width 0.25) (layer "F.Cu") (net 5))
 (segment (start 124.399 97.254) (end 125.175 98.03) (width 0.25) (layer "F.Cu") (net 5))
 (segment (start 125.875 95.145) (end 125.875 97.33) (width 0.25) (layer "F.Cu") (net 5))
 (segment (start 140.79 81.83) (end 135.205686 81.83) (width 0.25) (layer "F.Cu") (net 35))
 (segment (start 135.205686 81.83) (end 133.193402 83.842284) (width 0.25) (layer "F.Cu") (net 35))
 (segment (start 134.890458 85.53934) (end 136.87934 85.53934) (width 0.25) (layer "F.Cu") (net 32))
 (segment (start 136.87934 85.53934) (end 140.79 89.45) (width 0.25) (layer "F.Cu") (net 32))
 (segment (start 130.93066 94.699056) (end 130.93066 91.620458) (width 0.25) (layer "F.Cu") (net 27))
 (segment (start 139.133 96.175) (end 139.133 97.038225) (width 0.25) (layer "F.Cu") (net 27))
 (segment (start 140.74 94.568) (end 139.133 96.175) (width 0.25) (layer "F.Cu") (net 27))
 (segment (start 140.74 94.53) (end 140.74 94.568) (width 0.25) (layer "F.Cu") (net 27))
 (segment (start 137.965225 98.206) (end 134.437604 98.206) (width 0.25) (layer "F.Cu") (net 27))
 (segment (start 139.133 97.038225) (end 137.965225 98.206) (width 0.25) (layer "F.Cu") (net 27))
 (segment (start 134.437604 98.206) (end 130.93066 94.699056) (width 0.25) (layer "F.Cu") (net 27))
 (segment (start 136.614314 79.29) (end 132.627716 83.276598) (width 0.25) (layer "F.Cu") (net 36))
 (segment (start 140.79 79.29) (end 136.614314 79.29) (width 0.25) (layer "F.Cu") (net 36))
 (segment (start 127.864702 91.433725) (end 127.864702 94.354702) (width 0.25) (layer "F.Cu") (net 6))
 (segment (start 138.894 105.384) (end 140.74 107.23) (width 0.25) (layer "F.Cu") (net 6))
 (segment (start 128.243654 91.054773) (end 127.864702 91.433725) (width 0.25) (layer "F.Cu") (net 6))
 (segment (start 134.06 107.11) (end 134.06 105.91) (width 0.25) (layer "F.Cu") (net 6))
 (segment (start 134.06 105.91) (end 134.586 105.384) (width 0.25) (layer "F.Cu") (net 6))
 (segment (start 134.586 105.384) (end 138.894 105.384) (width 0.25) (layer "F.Cu") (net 6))
 (segment (start 127.864702 94.354702) (end 140.74 107.23) (width 0.25) (layer "F.Cu") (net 6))
 (segment (start 140.74 97.07) (end 139.154 98.656) (width 0.25) (layer "F.Cu") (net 41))
 (segment (start 139.154 98.656) (end 134.251208 98.656) (width 0.25) (layer "F.Cu") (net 41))
 (segment (start 129.24 93.644792) (end 129.24 92.051118) (width 0.25) (layer "F.Cu") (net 41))
 (segment (start 134.251208 98.656) (end 129.24 93.644792) (width 0.25) (layer "F.Cu") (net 41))
 (segment (start 129.24 92.051118) (end 128.80934 91.620458) (width 0.25) (layer "F.Cu") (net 41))
 (segment (start 134.367056 83.8) (end 140.22 83.8) (width 0.25) (layer "F.Cu") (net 34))
 (segment (start 140.22 83.8) (end 140.79 84.37) (width 0.25) (layer "F.Cu") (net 34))
 (segment (start 133.759087 84.407969) (end 134.367056 83.8) (width 0.25) (layer "F.Cu") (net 34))
 (segment (start 119.83 91.91) (end 124.849542 86.890458) (width 0.25) (layer "F.Cu") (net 16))
 (segment (start 124.849542 86.890458) (end 124.849542 85.53934) (width 0.25) (layer "F.Cu") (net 16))
 (segment (start 124.451 88.059202) (end 124.849542 87.66066) (width 0.25) (layer "F.Cu") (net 15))
 (segment (start 124.451 89.779) (end 124.451 88.059202) (width 0.25) (layer "F.Cu") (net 15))
 (segment (start 119.78 94.45) (end 124.451 89.779) (width 0.25) (layer "F.Cu") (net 15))
 (segment (start 130.298 105.190775) (end 128.98 106.508775) (width 0.25) (layer "F.Cu") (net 8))
 (segment (start 124.657 99.53) (end 126.399016 101.272016) (width 0.25) (layer "F.Cu") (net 8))
 (segment (start 128.98 106.508775) (end 128.98 107.11) (width 0.25) (layer "F.Cu") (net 8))
 (segment (start 130.298 103.370242) (end 130.298 105.190775) (width 0.25) (layer "F.Cu") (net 8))
 (segment (start 126.399016 101.272016) (end 128.199774 101.272016) (width 0.25) (layer "F.Cu") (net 8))
 (segment (start 119.78 99.53) (end 124.657 99.53) (width 0.25) (layer "F.Cu") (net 8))
 (segment (start 128.199774 101.272016) (end 130.298 103.370242) (width 0.25) (layer "F.Cu") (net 8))
 (segment (start 123.678518 85.521482) (end 123.678518 85.188668) (width 0.25) (layer "F.Cu") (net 17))
 (segment (start 125.036275 84.594702) (end 125.415227 84.973654) (width 0.25) (layer "F.Cu") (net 17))
 (segment (start 119.83 89.37) (end 123.678518 85.521482) (width 0.25) (layer "F.Cu") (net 17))
 (segment (start 123.678518 85.188668) (end 124.272484 84.594702) (width 0.25) (layer "F.Cu") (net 17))
 (segment (start 124.272484 84.594702) (end 125.036275 84.594702) (width 0.25) (layer "F.Cu") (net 17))
 (segment (start 122.1 82.02) (end 119.83 84.29) (width 0.25) (layer "F.Cu") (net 18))
 (segment (start 122.571604 76.77) (end 122.1 77.241604) (width 0.25) (layer "F.Cu") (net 18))
 (segment (start 129.25934 77.752944) (end 128.276396 76.77) (width 0.25) (layer "F.Cu") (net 18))
 (segment (start 122.1 77.241604) (end 122.1 82.02) (width 0.25) (layer "F.Cu") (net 18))
 (segment (start 130.93066 81.579542) (end 129.25934 79.908222) (width 0.25) (layer "F.Cu") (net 18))
 (segment (start 129.25934 79.908222) (end 129.25934 77.752944) (width 0.25) (layer "F.Cu") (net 18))
 (segment (start 128.276396 76.77) (end 122.571604 76.77) (width 0.25) (layer "F.Cu") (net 18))
 (segment (start 127.27 77.938) (end 127.914 77.294) (width 0.25) (layer "F.Cu") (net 3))
 (segment (start 127.27 78.095) (end 127.27 77.938) (width 0.25) (layer "F.Cu") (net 3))
 (segment (start 128.80934 78.18934) (end 128.80934 81.579542) (width 0.25) (layer "F.Cu") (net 3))
 (segment (start 127.914 77.294) (end 128.80934 78.18934) (width 0.25) (layer "F.Cu") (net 3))
 (segment (start 119.83 86.83) (end 122.684 83.976) (width 0.25) (layer "F.Cu") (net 3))
 (segment (start 122.684 77.294) (end 127.914 77.294) (width 0.25) (layer "F.Cu") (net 3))
 (segment (start 122.684 77.854) (end 122.59 77.76) (width 0.25) (layer "F.Cu") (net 3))
 (segment (start 122.59 77.388) (end 122.684 77.294) (width 0.25) (layer "F.Cu") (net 3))
 (segment (start 122.59 77.76) (end 122.59 77.388) (width 0.25) (layer "F.Cu") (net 3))
 (segment (start 122.684 83.976) (end 122.684 77.854) (width 0.25) (layer "F.Cu") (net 3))
 (segment (start 124.902 88.739573) (end 124.902 89.96581) (width 0.25) (layer "F.Cu") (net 14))
 (segment (start 125.415227 88.226346) (end 124.902 88.739573) (width 0.25) (layer "F.Cu") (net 14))
 (segment (start 124.902 89.96581) (end 121.056 93.81181) (width 0.25) (layer "F.Cu") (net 14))
 (segment (start 121.056 95.714) (end 119.78 96.99) (width 0.25) (layer "F.Cu") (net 14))
 (segment (start 121.056 93.81181) (end 121.056 95.714) (width 0.25) (layer "F.Cu") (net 14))
 (segment (start 129.70934 78.58934) (end 132.06 80.94) (width 0.25) (layer "F.Cu") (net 19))
 (segment (start 128.462792 76.32) (end 129.70934 77.566548) (width 0.25) (layer "F.Cu") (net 19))
 (segment (start 121.4 77.305208) (end 122.385208 76.32) (width 0.25) (layer "F.Cu") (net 19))
 (segment (start 132.06 81.581573) (end 131.496346 82.145227) (width 0.25) (layer "F.Cu") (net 19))
 (segment (start 119.83 81.75) (end 119.88 81.75) (width 0.25) (layer "F.Cu") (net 19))
 (segment (start 121.4 80.23) (end 121.4 77.305208) (width 0.25) (layer "F.Cu") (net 19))
 (segment (start 119.88 81.75) (end 121.4 80.23) (width 0.25) (layer "F.Cu") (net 19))
 (segment (start 132.06 80.94) (end 132.06 81.581573) (width 0.25) (layer "F.Cu") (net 19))
 (segment (start 129.70934 77.566548) (end 129.70934 78.58934) (width 0.25) (layer "F.Cu") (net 19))
 (segment (start 122.385208 76.32) (end 128.462792 76.32) (width 0.25) (layer "F.Cu") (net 19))
 (segment (start 127.809188 75.69) (end 128.92 75.69) (width 0.25) (layer "F.Cu") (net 20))
 (segment (start 132.899188 81.873756) (end 132.062031 82.710913) (width 0.25) (layer "F.Cu") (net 20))
 (segment (start 127.489188 75.37) (end 127.809188 75.69) (width 0.25) (layer "F.Cu") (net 20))
 (segment (start 119.83 79.21) (end 119.83 78.06) (width 0.25) (layer "F.Cu") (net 20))
 (segment (start 122.52 75.37) (end 127.489188 75.37) (width 0.25) (layer "F.Cu") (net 20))
 (segment (start 119.83 78.06) (end 122.52 75.37) (width 0.25) (layer "F.Cu") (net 20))
 (segment (start 132.899188 79.669188) (end 132.899188 81.873756) (width 0.25) (layer "F.Cu") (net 20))
 (segment (start 128.92 75.69) (end 132.899188 79.669188) (width 0.25) (layer "F.Cu") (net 20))
 (segment (start 129.83 83.731573) (end 129.83 87.125686) (width 0.25) (layer "F.Cu") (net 30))
 (segment (start 128.243654 82.145227) (end 129.83 83.731573) (width 0.25) (layer "F.Cu") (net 30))
 (segment (start 129.83 87.125686) (end 132.627716 89.923402) (width 0.25) (layer "F.Cu") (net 30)))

